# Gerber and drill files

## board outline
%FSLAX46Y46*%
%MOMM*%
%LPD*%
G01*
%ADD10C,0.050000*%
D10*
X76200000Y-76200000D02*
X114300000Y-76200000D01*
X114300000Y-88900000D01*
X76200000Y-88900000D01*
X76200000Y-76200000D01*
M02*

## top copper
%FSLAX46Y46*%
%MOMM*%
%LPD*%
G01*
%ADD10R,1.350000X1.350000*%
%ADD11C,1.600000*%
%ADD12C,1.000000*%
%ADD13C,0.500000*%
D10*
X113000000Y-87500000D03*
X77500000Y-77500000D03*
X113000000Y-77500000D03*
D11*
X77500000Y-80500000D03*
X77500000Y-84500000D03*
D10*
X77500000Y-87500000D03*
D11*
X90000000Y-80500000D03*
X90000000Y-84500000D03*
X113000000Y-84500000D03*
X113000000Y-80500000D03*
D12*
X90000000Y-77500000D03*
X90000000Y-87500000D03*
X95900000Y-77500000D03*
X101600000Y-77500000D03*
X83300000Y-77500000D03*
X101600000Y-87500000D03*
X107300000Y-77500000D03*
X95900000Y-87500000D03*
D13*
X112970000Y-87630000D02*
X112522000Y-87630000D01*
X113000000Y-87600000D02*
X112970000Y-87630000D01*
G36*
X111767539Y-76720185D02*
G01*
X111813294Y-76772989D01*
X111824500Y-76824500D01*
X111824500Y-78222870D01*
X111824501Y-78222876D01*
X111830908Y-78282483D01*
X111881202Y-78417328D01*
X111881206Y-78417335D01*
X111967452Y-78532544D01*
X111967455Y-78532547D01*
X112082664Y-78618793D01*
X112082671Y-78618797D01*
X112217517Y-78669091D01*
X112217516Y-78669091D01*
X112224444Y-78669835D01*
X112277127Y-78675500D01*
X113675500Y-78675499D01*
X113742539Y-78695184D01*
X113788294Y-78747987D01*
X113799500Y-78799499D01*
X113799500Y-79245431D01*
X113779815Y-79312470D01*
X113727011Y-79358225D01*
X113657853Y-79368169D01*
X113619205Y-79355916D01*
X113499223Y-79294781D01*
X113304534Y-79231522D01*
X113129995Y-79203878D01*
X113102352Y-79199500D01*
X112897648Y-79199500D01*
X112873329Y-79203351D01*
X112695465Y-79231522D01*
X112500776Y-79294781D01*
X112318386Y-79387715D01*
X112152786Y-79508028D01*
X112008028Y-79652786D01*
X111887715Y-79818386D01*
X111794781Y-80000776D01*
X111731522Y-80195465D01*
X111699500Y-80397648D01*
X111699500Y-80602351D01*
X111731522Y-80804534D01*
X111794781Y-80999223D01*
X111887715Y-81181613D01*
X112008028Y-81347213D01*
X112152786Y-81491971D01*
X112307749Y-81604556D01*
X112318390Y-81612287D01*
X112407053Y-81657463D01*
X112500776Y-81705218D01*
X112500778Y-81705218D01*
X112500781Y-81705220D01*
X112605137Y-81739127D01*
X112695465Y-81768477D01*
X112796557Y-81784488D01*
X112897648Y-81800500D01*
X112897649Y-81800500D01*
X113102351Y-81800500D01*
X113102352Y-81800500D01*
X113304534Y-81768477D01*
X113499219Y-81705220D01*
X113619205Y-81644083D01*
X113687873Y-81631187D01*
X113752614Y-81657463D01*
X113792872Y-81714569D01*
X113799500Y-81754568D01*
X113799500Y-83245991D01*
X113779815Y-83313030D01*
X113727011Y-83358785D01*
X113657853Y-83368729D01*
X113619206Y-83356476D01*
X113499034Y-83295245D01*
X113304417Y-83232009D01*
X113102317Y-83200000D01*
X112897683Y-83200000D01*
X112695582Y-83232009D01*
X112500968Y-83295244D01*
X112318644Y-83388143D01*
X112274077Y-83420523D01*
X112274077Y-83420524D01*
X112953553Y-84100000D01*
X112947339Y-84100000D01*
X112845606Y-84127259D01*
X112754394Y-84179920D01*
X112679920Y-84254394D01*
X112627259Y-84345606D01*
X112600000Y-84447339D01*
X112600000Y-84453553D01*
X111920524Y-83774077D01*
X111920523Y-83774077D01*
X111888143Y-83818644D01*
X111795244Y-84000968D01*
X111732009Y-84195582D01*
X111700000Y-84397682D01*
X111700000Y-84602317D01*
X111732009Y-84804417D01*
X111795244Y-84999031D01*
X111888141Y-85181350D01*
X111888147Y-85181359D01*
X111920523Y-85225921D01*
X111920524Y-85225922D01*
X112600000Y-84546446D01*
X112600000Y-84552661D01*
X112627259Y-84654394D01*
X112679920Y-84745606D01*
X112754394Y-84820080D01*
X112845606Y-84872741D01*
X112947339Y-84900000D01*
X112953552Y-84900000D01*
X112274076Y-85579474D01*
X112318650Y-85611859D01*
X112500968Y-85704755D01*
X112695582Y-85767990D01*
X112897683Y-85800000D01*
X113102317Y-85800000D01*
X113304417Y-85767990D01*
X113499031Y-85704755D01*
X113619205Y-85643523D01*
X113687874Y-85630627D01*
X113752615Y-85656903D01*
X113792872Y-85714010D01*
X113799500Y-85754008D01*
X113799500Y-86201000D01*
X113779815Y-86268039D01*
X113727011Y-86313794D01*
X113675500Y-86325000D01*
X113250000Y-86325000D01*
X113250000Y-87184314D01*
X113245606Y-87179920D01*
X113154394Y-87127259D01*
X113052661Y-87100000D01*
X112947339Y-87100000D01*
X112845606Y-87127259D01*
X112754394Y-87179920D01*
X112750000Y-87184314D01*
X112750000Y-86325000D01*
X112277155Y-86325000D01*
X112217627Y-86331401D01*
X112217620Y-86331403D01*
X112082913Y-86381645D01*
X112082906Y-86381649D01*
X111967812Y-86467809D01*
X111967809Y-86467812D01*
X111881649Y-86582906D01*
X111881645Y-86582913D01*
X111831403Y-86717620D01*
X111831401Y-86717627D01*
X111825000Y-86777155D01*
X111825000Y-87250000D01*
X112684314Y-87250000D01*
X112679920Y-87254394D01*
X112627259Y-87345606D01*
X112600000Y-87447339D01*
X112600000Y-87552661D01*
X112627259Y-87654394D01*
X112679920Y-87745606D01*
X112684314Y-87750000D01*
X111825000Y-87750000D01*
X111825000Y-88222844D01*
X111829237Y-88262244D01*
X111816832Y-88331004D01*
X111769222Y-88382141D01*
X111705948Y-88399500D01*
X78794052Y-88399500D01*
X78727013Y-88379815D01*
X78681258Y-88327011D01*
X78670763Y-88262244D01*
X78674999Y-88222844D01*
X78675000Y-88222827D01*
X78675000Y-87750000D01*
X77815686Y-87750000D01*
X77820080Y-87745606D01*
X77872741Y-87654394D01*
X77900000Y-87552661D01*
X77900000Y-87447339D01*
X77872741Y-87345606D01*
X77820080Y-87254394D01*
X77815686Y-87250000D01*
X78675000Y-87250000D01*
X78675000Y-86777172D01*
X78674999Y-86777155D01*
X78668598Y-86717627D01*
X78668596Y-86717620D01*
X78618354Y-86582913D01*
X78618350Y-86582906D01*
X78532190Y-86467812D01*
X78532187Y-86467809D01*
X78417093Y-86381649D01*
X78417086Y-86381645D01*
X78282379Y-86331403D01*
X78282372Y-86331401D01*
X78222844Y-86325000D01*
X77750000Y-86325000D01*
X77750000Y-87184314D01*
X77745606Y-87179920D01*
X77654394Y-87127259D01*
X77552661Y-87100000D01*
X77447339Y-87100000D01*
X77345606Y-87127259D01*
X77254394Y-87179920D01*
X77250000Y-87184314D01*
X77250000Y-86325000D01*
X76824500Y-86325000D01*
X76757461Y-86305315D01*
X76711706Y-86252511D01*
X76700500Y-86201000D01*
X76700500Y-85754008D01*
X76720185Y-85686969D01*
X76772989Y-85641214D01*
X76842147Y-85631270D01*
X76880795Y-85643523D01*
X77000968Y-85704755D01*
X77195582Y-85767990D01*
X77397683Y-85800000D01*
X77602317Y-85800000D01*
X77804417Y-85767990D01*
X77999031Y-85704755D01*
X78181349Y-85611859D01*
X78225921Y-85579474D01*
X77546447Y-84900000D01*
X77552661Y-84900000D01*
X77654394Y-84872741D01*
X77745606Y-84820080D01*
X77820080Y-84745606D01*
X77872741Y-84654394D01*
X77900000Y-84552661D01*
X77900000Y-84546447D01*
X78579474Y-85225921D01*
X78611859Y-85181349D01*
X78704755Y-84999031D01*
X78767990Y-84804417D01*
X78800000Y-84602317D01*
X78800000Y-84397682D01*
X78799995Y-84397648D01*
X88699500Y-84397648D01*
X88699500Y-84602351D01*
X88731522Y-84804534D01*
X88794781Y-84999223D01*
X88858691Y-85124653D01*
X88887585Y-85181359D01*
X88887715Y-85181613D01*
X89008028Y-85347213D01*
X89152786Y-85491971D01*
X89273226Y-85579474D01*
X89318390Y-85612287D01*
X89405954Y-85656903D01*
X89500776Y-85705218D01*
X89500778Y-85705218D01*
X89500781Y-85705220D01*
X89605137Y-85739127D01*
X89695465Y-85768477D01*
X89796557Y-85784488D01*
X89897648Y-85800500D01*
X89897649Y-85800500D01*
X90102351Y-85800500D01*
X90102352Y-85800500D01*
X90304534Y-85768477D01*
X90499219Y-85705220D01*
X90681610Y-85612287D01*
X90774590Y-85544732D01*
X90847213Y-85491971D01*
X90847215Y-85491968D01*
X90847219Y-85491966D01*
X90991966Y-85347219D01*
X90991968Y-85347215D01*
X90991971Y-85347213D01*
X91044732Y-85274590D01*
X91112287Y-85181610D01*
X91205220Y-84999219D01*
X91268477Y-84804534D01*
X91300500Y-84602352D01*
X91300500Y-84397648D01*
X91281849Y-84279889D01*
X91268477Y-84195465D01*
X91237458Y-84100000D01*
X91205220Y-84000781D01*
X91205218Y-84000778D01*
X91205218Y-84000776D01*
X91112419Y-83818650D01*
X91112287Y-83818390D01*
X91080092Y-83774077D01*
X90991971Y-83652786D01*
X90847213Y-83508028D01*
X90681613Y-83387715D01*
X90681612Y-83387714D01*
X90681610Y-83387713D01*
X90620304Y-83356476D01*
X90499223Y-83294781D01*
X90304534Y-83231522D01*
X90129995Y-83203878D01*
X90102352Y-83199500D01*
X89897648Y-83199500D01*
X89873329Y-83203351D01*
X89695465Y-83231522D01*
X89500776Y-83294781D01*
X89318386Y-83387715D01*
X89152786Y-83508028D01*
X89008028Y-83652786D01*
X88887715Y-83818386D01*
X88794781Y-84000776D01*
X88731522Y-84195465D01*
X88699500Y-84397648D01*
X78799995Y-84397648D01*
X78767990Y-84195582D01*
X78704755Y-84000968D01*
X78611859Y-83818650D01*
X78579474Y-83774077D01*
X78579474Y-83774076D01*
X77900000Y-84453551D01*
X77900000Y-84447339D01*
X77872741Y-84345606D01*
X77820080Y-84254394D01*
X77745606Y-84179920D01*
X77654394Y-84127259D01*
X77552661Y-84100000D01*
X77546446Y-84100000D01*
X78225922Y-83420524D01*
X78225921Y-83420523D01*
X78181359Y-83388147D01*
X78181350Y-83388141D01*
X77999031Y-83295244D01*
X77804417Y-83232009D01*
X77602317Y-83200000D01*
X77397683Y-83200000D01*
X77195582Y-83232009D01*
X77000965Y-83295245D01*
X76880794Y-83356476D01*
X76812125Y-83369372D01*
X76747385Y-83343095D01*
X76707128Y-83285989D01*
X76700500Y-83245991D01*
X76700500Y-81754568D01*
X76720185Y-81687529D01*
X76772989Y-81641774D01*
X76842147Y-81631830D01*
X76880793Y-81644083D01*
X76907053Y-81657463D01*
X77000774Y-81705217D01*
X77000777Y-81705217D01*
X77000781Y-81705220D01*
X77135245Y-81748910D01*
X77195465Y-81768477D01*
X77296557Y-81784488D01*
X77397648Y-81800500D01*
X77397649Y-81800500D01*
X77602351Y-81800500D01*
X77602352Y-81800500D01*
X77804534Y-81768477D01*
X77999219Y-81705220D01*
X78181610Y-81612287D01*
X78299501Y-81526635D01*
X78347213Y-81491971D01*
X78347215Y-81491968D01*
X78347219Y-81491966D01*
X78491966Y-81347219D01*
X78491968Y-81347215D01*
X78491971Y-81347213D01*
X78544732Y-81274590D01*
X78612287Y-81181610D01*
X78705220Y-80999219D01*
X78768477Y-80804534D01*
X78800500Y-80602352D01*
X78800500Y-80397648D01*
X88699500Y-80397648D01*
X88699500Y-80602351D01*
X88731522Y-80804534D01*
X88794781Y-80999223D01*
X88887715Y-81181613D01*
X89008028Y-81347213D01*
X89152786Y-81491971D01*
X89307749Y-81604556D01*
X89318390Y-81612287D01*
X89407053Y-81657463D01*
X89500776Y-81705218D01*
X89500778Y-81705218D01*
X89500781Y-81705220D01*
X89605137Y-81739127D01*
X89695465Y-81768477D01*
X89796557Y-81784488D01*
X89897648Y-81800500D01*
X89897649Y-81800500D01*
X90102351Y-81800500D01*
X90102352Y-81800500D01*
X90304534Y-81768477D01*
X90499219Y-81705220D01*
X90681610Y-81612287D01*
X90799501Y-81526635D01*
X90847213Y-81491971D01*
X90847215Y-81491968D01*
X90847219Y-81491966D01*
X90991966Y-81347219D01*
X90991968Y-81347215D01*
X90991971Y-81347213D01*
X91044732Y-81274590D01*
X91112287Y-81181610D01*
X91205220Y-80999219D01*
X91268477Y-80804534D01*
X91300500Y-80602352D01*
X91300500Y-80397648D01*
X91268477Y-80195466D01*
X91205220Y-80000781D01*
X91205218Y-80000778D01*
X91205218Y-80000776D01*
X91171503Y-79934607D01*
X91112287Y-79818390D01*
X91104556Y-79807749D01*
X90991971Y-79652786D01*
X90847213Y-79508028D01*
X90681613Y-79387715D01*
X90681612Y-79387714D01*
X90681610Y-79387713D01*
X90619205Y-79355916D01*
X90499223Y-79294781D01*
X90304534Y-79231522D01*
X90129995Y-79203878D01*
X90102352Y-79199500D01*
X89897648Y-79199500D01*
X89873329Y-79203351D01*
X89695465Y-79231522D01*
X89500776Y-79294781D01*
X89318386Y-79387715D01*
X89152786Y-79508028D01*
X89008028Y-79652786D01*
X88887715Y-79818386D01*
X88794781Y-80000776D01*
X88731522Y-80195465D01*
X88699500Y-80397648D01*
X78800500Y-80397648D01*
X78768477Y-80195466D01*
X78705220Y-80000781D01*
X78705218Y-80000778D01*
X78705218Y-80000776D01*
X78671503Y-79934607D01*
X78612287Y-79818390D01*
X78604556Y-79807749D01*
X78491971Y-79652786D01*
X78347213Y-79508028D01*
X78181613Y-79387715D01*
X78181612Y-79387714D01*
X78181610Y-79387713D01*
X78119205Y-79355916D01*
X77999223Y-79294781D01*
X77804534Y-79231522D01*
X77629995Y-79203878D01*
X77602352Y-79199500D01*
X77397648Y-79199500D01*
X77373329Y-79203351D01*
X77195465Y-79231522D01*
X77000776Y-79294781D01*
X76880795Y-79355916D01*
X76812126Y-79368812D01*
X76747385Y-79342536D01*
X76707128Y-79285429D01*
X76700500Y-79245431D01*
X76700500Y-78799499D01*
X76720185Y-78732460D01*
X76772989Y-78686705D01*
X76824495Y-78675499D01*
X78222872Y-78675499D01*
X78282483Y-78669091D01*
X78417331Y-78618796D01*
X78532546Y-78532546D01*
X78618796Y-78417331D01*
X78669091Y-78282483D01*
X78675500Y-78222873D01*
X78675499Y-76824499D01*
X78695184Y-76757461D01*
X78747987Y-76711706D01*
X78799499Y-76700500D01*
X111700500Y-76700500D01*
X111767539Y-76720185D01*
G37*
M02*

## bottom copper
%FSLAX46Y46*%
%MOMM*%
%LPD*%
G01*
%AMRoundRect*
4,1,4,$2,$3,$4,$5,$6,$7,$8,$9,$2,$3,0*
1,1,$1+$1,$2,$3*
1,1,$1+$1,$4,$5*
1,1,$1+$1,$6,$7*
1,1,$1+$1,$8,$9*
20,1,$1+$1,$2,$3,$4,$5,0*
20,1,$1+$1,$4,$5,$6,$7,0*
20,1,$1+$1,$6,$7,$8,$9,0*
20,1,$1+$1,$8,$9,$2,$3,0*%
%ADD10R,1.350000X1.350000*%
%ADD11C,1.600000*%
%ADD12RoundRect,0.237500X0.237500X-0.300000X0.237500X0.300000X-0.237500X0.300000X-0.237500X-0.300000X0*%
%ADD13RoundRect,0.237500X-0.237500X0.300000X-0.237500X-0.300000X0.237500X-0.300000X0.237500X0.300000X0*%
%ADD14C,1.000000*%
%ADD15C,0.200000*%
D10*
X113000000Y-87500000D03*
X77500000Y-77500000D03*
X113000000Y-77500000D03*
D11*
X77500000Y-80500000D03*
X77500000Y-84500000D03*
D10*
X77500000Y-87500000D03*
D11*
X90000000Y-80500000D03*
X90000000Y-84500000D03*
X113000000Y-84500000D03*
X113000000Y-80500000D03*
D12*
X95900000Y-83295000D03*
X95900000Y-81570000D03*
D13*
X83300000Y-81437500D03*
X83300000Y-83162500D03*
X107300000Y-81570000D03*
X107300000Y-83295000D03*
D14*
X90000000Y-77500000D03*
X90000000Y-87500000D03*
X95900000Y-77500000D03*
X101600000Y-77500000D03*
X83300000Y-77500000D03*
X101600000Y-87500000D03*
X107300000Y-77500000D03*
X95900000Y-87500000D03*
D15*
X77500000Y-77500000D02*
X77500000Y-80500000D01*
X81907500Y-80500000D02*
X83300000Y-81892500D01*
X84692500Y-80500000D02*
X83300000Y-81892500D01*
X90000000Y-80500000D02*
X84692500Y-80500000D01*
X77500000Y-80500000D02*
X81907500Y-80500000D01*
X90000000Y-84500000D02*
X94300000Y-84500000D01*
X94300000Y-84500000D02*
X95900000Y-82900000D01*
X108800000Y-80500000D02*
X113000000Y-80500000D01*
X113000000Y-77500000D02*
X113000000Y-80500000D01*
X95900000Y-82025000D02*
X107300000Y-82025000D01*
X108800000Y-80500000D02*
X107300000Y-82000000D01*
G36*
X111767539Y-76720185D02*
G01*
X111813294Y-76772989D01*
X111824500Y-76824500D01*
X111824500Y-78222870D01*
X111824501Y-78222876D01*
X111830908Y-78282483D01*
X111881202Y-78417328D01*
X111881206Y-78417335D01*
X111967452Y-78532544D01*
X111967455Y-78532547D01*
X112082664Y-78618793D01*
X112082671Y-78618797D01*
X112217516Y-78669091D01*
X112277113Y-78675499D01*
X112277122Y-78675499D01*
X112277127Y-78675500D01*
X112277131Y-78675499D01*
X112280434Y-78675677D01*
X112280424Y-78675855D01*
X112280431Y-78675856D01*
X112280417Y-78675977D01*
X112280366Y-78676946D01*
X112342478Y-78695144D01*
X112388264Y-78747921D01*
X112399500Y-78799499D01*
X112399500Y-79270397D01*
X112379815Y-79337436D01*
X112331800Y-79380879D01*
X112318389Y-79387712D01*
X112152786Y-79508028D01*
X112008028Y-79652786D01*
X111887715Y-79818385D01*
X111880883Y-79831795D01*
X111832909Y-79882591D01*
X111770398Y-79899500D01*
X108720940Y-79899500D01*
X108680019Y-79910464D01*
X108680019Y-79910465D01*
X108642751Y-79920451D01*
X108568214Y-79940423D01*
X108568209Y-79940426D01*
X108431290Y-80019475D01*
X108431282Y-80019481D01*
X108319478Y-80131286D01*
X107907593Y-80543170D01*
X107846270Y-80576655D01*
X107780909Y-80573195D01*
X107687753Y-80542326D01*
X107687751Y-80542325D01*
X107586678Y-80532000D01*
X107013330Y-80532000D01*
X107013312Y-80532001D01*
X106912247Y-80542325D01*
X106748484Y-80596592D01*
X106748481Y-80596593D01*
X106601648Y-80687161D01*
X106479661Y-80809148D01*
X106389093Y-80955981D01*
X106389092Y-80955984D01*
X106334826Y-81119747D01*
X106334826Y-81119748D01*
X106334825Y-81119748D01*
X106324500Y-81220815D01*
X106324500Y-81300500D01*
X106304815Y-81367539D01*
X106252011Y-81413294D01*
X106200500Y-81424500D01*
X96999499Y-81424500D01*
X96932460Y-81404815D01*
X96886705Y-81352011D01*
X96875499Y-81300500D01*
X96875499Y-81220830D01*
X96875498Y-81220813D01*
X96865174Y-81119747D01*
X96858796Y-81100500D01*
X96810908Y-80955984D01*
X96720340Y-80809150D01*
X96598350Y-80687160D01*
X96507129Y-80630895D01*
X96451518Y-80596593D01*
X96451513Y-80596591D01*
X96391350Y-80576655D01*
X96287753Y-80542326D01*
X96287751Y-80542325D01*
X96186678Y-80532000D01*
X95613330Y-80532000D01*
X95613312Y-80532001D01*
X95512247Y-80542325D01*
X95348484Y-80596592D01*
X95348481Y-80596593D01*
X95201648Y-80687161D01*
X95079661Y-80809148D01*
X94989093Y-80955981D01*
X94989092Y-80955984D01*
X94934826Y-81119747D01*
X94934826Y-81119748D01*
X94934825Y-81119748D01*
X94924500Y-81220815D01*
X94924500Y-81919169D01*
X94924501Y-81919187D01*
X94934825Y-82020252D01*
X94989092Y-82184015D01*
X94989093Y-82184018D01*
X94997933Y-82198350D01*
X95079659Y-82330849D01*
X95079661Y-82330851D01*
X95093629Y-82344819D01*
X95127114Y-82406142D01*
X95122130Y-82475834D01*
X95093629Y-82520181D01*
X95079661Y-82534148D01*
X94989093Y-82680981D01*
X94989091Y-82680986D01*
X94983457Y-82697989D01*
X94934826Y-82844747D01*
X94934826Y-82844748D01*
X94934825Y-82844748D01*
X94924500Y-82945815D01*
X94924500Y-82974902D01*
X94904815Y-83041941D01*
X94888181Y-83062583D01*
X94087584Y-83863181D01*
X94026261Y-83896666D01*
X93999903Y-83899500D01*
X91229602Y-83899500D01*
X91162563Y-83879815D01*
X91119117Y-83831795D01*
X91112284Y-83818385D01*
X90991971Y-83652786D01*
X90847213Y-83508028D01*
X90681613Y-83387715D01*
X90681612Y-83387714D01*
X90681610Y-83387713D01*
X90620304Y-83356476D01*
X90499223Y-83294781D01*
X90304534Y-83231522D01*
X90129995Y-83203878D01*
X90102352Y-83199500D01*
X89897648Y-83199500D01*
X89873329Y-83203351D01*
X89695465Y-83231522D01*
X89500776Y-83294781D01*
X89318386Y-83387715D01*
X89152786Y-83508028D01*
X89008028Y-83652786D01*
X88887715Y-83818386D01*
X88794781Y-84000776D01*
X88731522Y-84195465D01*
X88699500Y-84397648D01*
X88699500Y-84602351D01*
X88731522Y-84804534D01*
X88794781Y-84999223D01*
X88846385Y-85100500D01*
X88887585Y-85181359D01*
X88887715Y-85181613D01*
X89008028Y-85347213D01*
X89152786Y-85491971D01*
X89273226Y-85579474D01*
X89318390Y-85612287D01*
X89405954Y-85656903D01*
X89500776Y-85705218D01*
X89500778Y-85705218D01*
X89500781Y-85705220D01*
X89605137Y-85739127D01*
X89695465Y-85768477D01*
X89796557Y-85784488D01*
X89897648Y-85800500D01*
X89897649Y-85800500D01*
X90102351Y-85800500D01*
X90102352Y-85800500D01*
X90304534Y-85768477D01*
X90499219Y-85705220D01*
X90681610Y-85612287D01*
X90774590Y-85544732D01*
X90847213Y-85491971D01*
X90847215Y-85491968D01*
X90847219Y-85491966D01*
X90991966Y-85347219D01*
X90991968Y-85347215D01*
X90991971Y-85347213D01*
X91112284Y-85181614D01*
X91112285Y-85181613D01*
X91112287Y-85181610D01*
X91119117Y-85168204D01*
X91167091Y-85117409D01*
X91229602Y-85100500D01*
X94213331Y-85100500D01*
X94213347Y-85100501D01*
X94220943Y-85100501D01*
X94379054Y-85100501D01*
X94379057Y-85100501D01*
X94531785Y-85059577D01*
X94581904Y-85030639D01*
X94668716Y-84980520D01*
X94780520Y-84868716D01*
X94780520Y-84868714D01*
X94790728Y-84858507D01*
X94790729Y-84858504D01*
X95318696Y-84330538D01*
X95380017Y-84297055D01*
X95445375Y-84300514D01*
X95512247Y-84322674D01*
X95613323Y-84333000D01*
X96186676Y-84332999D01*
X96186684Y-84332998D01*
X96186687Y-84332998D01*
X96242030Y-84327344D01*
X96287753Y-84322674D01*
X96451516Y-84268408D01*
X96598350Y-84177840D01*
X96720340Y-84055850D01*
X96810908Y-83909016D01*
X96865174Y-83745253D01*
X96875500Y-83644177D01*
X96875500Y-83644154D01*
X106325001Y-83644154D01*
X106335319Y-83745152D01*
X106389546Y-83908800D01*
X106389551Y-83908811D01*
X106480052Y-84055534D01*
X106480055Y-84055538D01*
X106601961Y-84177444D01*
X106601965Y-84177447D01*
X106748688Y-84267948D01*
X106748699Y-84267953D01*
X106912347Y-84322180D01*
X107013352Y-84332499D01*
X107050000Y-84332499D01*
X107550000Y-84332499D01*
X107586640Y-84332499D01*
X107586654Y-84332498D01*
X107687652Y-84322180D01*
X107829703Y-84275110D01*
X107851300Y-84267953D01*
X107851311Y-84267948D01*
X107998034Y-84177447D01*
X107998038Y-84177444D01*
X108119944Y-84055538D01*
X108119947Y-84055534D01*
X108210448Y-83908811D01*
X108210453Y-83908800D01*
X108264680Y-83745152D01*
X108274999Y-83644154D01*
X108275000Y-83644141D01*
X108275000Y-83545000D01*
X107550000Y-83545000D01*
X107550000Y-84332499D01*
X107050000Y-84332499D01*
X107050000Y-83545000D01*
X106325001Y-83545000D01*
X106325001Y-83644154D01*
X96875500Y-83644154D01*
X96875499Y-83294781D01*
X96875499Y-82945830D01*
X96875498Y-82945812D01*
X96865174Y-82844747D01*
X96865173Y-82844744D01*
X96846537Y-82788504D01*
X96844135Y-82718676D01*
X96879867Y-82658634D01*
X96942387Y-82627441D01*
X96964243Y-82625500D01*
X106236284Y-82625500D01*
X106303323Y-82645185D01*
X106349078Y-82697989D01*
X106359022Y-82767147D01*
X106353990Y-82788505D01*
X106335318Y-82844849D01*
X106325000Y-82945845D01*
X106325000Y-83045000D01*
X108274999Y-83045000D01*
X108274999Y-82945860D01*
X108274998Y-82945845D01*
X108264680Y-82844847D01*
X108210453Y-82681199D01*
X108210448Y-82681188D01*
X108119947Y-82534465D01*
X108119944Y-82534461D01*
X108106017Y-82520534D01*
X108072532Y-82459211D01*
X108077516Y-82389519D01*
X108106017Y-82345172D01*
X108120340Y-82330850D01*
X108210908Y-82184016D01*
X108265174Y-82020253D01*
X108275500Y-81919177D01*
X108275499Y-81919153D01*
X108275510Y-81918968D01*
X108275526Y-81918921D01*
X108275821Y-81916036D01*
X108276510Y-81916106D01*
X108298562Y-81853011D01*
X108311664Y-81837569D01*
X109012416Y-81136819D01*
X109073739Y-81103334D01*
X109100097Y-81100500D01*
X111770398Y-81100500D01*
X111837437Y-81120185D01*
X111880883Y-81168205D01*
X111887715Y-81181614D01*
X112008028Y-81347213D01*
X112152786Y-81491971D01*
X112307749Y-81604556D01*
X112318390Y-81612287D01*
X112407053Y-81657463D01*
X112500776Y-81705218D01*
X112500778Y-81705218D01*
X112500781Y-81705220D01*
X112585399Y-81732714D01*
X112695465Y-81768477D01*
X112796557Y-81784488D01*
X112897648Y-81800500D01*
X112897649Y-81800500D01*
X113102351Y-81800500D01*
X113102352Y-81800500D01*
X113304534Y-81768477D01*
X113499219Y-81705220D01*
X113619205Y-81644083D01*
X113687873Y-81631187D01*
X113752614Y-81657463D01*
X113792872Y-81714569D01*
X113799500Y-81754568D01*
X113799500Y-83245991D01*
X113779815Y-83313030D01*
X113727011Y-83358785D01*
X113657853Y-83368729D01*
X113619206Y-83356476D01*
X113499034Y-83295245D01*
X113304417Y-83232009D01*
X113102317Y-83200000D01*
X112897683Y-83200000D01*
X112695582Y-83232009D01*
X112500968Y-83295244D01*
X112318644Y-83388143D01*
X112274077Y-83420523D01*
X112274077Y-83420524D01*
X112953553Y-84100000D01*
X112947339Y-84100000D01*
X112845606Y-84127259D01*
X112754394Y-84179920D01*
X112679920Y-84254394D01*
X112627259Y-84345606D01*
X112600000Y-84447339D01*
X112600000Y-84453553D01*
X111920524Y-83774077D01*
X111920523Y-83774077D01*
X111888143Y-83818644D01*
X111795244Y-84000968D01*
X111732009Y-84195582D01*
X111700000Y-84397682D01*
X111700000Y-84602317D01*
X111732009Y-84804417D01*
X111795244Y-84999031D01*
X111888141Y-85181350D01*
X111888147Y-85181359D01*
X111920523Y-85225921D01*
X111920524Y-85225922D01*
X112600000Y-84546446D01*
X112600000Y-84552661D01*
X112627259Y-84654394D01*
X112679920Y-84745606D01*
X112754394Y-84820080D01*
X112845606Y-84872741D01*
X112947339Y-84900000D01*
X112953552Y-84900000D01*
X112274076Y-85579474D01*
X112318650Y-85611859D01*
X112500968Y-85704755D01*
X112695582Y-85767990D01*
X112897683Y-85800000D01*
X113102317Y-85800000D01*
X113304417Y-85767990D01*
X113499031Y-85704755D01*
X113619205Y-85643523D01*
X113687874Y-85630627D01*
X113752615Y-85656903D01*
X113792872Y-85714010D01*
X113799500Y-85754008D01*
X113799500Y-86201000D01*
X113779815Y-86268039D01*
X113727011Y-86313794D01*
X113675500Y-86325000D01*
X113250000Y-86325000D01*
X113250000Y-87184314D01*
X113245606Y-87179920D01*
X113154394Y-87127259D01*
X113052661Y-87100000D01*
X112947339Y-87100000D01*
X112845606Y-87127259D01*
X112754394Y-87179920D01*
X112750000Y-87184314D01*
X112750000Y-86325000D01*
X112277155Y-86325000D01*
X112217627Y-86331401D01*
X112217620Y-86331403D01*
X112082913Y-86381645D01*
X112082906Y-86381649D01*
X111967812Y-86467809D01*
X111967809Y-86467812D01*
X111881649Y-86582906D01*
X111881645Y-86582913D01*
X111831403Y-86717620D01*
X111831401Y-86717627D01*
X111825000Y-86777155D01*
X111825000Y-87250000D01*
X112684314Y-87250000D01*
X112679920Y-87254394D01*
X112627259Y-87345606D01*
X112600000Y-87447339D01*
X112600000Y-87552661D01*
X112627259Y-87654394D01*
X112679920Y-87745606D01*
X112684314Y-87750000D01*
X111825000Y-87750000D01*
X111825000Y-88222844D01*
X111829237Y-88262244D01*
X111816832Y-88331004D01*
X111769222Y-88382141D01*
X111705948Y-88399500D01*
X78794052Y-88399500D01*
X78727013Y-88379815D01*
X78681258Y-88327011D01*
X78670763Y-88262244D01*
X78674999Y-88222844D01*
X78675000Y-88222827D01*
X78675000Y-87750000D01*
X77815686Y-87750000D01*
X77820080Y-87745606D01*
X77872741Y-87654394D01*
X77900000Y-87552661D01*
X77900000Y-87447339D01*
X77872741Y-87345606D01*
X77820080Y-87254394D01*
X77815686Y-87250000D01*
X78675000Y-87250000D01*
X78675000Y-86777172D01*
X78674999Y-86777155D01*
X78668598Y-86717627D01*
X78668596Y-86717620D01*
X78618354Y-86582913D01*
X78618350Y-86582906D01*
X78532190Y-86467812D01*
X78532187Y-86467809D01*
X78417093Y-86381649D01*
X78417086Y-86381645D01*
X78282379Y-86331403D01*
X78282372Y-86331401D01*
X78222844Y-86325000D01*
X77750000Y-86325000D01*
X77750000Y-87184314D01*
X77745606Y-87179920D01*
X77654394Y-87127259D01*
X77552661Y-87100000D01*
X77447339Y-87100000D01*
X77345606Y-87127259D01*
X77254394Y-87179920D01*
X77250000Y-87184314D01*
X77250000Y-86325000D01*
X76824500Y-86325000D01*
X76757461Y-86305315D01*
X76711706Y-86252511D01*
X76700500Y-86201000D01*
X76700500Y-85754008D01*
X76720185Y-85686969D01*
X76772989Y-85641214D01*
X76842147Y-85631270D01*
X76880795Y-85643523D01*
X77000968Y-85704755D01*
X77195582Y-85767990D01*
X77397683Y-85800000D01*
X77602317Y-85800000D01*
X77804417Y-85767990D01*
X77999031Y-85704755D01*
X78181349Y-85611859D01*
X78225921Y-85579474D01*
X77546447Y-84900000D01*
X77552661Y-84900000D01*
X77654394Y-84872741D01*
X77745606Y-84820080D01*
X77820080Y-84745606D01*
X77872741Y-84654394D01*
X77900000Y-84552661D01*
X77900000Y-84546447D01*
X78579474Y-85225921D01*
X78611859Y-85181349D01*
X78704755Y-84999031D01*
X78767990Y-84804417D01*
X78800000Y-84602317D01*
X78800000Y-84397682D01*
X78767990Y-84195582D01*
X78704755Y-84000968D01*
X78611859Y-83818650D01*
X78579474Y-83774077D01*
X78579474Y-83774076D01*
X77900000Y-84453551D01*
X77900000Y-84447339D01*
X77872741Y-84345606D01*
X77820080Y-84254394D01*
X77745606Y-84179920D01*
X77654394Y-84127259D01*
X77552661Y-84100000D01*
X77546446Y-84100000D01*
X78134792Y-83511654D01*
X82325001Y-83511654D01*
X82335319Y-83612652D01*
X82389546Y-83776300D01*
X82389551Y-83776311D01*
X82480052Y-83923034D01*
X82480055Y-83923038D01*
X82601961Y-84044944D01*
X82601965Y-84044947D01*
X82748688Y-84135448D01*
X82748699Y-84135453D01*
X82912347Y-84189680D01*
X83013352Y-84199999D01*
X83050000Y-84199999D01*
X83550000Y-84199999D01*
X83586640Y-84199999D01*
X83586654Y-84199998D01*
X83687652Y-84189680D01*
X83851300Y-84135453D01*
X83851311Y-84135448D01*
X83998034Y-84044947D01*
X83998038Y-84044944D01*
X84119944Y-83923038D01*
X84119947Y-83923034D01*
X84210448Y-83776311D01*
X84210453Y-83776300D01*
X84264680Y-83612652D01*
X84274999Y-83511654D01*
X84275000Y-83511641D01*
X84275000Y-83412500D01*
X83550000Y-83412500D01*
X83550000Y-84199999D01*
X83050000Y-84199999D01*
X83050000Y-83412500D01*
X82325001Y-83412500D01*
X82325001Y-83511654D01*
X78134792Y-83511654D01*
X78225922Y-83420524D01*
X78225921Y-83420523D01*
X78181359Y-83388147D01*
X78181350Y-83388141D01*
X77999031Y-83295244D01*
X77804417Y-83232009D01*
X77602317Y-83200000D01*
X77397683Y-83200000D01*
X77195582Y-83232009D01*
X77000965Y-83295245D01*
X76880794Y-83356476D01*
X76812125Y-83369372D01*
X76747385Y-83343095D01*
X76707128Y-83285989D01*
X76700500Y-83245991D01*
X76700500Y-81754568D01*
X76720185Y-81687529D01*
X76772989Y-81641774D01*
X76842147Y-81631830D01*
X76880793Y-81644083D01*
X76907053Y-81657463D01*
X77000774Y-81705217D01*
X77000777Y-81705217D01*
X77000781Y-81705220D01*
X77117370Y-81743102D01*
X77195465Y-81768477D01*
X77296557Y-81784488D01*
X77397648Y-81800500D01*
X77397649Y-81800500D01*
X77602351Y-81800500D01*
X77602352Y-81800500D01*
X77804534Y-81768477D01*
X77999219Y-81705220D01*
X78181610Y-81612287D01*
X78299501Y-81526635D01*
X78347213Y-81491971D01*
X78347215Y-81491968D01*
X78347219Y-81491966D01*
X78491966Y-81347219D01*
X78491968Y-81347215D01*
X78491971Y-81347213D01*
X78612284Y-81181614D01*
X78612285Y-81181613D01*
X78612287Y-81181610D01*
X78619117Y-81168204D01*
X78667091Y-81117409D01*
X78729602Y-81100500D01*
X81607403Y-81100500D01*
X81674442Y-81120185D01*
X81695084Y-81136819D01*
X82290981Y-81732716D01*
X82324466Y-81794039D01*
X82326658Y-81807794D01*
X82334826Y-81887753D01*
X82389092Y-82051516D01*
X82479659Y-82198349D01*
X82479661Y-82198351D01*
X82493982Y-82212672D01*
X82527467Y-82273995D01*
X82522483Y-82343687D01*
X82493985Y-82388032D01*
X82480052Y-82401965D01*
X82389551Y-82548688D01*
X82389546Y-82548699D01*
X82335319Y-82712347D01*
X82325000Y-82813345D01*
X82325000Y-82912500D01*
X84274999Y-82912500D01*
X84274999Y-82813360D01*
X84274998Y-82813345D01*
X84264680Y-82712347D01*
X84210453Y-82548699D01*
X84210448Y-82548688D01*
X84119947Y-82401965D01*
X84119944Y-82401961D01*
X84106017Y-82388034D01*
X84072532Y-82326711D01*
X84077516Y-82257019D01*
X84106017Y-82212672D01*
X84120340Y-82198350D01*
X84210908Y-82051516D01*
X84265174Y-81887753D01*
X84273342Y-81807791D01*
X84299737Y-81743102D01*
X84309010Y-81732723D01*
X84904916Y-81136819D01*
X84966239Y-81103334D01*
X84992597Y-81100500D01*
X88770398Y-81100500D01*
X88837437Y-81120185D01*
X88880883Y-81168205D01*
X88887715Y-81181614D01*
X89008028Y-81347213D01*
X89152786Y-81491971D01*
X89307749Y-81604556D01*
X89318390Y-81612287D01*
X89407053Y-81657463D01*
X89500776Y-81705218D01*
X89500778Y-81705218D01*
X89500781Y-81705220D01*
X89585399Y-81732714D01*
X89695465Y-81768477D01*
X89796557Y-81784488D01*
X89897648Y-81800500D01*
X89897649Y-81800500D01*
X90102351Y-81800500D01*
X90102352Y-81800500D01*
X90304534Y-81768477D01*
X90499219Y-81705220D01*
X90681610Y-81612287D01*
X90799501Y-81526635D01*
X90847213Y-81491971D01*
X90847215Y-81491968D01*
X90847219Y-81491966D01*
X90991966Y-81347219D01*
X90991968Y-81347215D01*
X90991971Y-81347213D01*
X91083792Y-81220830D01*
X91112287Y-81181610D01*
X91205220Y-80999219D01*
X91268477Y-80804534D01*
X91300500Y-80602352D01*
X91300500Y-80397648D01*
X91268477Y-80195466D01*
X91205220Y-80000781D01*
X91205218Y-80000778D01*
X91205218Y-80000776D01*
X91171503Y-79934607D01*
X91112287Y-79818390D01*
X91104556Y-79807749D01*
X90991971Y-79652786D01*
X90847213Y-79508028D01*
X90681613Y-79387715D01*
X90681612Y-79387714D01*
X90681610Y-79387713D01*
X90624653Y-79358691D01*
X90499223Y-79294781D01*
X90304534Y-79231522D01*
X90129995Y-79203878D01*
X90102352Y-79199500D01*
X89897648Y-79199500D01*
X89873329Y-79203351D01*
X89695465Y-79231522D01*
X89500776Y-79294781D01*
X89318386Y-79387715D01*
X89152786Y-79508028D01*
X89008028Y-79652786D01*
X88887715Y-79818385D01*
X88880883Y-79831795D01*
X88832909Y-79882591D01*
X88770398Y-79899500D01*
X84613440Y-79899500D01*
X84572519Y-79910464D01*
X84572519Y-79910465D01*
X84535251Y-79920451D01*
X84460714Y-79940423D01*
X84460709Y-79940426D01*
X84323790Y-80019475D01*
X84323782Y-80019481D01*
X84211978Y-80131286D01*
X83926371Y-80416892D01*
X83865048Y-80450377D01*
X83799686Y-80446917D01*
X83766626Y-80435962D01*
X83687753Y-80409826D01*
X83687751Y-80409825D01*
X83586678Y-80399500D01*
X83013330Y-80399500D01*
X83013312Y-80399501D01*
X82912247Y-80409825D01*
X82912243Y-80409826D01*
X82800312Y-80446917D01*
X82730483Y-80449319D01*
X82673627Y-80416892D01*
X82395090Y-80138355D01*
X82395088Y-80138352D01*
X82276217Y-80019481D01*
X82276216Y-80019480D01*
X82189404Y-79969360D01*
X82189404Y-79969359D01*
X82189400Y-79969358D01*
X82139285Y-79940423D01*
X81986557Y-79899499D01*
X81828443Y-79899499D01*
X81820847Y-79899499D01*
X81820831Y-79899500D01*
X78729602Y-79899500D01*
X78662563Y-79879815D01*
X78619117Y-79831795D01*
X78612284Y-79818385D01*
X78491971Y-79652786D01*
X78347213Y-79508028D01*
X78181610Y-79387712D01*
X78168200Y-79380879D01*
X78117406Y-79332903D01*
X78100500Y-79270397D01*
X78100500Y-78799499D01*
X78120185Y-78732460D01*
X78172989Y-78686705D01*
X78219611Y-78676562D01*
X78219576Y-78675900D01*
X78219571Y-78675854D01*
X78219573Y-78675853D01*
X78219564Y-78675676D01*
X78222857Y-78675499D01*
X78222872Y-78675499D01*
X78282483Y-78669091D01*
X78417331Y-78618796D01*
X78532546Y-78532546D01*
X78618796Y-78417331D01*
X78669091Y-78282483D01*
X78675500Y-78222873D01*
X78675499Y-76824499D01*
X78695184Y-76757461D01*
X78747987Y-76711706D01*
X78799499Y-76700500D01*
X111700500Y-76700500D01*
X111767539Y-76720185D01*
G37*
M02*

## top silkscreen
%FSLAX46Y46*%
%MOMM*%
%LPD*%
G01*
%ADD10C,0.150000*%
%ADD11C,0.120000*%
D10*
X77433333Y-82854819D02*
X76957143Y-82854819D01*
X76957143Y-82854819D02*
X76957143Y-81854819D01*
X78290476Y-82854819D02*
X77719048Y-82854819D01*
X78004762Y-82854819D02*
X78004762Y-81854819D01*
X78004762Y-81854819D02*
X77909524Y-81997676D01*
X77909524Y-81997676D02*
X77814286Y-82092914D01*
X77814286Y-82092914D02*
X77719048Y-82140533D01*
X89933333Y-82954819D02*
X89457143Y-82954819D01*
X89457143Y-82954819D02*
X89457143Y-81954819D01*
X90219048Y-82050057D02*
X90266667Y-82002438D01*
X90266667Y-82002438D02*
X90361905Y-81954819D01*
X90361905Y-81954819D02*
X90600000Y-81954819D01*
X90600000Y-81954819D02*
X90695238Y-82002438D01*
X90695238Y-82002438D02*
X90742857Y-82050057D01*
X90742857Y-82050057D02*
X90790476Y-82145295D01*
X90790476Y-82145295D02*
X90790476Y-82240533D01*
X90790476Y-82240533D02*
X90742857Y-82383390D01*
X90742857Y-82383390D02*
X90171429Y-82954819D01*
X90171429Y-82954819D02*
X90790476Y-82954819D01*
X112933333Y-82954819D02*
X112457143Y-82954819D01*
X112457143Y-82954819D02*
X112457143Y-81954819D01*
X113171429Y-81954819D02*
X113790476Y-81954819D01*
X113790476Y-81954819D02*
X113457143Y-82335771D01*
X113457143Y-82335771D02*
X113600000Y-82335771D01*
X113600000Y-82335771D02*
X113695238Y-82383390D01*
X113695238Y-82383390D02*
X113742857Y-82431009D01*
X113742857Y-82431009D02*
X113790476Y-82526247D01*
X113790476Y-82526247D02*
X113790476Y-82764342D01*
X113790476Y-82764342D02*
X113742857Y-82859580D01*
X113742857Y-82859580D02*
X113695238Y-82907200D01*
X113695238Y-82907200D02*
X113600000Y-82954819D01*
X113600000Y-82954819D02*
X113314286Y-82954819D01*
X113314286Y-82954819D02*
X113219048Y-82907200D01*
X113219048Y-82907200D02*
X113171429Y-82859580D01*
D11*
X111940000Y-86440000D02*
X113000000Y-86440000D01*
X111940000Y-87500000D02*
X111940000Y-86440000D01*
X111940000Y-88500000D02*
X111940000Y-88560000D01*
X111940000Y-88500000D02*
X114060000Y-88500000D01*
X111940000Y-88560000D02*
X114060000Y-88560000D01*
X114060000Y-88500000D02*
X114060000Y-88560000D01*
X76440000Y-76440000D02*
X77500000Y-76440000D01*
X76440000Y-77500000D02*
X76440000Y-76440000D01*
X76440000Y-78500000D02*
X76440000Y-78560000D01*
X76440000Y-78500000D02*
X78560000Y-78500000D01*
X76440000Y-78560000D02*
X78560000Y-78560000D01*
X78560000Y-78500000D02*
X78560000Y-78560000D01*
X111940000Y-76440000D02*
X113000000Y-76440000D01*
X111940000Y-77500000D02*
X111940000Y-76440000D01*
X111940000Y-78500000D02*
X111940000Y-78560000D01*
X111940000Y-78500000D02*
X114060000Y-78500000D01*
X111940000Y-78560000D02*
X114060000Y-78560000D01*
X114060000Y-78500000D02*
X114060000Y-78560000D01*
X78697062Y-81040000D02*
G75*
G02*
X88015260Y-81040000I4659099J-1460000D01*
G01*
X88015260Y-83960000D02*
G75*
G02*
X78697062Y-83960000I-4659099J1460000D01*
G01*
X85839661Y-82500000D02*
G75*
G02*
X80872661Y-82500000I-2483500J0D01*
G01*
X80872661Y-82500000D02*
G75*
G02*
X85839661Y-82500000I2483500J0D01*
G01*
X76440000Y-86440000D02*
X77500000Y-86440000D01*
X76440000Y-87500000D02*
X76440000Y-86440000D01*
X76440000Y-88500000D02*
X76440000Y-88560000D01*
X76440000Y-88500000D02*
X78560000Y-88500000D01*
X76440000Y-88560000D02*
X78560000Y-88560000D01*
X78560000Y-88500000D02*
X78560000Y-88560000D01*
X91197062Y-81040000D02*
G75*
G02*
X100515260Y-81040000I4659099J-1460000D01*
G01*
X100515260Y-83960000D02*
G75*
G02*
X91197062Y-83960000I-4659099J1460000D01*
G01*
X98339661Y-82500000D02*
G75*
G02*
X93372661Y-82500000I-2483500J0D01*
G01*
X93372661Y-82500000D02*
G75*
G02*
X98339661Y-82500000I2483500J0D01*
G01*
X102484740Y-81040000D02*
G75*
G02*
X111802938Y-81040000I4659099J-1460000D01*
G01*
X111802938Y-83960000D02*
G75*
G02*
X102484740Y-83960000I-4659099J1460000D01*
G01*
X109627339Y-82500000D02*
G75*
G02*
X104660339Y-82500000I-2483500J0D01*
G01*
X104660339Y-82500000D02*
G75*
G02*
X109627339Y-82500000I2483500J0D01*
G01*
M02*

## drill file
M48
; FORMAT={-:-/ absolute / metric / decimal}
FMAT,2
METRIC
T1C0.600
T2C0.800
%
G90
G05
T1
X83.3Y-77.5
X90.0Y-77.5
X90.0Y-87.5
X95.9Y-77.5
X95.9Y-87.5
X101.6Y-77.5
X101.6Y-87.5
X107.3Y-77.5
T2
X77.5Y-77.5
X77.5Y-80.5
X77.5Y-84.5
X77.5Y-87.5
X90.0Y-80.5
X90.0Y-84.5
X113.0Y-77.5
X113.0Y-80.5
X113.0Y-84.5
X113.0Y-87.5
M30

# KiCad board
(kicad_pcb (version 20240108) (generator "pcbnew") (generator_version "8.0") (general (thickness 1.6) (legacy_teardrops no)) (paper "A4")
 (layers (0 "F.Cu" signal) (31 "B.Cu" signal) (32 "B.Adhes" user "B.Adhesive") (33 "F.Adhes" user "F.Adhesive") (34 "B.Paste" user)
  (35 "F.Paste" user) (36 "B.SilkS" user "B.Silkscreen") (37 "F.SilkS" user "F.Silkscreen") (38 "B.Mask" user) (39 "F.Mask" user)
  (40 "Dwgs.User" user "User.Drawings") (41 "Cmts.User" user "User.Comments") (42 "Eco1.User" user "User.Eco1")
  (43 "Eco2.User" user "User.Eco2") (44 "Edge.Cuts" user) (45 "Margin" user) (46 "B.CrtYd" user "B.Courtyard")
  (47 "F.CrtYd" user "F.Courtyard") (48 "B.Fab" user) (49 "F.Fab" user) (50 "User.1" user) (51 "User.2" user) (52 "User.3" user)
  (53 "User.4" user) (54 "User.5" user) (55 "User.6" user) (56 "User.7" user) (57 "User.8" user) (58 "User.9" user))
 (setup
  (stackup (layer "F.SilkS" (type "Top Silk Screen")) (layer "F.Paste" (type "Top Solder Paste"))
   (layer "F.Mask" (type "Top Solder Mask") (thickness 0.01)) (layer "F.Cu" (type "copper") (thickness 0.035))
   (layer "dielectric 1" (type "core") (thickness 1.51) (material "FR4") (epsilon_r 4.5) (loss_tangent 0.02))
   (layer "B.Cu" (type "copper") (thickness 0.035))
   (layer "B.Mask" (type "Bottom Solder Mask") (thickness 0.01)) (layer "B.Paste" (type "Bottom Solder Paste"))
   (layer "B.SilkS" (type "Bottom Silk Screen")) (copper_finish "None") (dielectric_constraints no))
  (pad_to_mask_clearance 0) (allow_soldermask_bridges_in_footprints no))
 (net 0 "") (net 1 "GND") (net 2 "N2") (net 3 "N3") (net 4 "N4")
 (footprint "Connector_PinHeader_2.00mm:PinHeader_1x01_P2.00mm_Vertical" (layer "F.Cu") (at 113 87.5)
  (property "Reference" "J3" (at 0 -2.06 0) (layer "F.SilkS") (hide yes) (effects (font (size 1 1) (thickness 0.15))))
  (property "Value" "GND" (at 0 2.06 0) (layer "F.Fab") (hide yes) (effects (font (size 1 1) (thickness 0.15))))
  (fp_line (start -1.06 -1.06) (end 0 -1.06) (stroke (width 0.12) (type solid)) (layer "F.SilkS"))
  (fp_line (start -1.06 0) (end -1.06 -1.06) (stroke (width 0.12) (type solid)) (layer "F.SilkS"))
  (fp_line (start -1.06 1) (end -1.06 1.06) (stroke (width 0.12) (type solid)) (layer "F.SilkS"))
  (fp_line (start -1.06 1) (end 1.06 1) (stroke (width 0.12) (type solid)) (layer "F.SilkS"))
  (fp_line (start -1.06 1.06) (end 1.06 1.06) (stroke (width 0.12) (type solid)) (layer "F.SilkS"))
  (fp_line (start 1.06 1) (end 1.06 1.06) (stroke (width 0.12) (type solid)) (layer "F.SilkS"))
  (pad "1" thru_hole rect (at 0 0) (size 1.35 1.35) (drill 0.8) (layers "*.Cu" "*.Mask") (remove_unused_layers no) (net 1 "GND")))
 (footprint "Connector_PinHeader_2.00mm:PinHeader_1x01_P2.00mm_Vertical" (layer "F.Cu") (at 77.5 77.5)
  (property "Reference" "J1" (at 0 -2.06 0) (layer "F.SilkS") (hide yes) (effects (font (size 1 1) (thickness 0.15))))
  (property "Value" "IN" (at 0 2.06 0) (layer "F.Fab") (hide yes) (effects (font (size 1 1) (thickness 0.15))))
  (fp_line (start -1.06 -1.06) (end 0 -1.06) (stroke (width 0.12) (type solid)) (layer "F.SilkS"))
  (fp_line (start -1.06 0) (end -1.06 -1.06) (stroke (width 0.12) (type solid)) (layer "F.SilkS"))
  (fp_line (start -1.06 1) (end -1.06 1.06) (stroke (width 0.12) (type solid)) (layer "F.SilkS"))
  (fp_line (start -1.06 1) (end 1.06 1) (stroke (width 0.12) (type solid)) (layer "F.SilkS"))
  (fp_line (start -1.06 1.06) (end 1.06 1.06) (stroke (width 0.12) (type solid)) (layer "F.SilkS"))
  (fp_line (start 1.06 1) (end 1.06 1.06) (stroke (width 0.12) (type solid)) (layer "F.SilkS"))
  (pad "1" thru_hole rect (at 0 0) (size 1.35 1.35) (drill 0.8) (layers "*.Cu" "*.Mask") (remove_unused_layers no) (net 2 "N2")))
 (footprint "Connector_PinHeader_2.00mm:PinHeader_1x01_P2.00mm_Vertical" (layer "F.Cu") (at 113 77.5)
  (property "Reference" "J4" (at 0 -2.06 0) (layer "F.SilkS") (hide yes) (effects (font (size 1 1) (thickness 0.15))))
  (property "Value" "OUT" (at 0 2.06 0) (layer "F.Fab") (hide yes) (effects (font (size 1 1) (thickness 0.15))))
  (fp_line (start -1.06 -1.06) (end 0 -1.06) (stroke (width 0.12) (type solid)) (layer "F.SilkS"))
  (fp_line (start -1.06 0) (end -1.06 -1.06) (stroke (width 0.12) (type solid)) (layer "F.SilkS"))
  (fp_line (start -1.06 1) (end -1.06 1.06) (stroke (width 0.12) (type solid)) (layer "F.SilkS"))
  (fp_line (start -1.06 1) (end 1.06 1) (stroke (width 0.12) (type solid)) (layer "F.SilkS"))
  (fp_line (start -1.06 1.06) (end 1.06 1.06) (stroke (width 0.12) (type solid)) (layer "F.SilkS"))
  (fp_line (start 1.06 1) (end 1.06 1.06) (stroke (width 0.12) (type solid)) (layer "F.SilkS"))
  (pad "1" thru_hole rect (at 0 0) (size 1.35 1.35) (drill 0.8) (layers "*.Cu" "*.Mask") (remove_unused_layers no) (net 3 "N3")))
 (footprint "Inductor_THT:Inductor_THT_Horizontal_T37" (layer "F.Cu") (at 77.5 82.5)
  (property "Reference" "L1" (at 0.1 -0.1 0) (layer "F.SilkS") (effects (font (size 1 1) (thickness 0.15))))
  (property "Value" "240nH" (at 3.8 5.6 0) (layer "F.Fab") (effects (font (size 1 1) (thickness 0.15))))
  (fp_arc (start 1.197062 -1.46) (mid 5.856161 -4.8825) (end 10.51526 -1.46) (stroke (width 0.12) (type solid)) (layer "F.SilkS"))
  (fp_arc (start 10.51526 1.46) (mid 5.856161 4.8825) (end 1.197062 1.46) (stroke (width 0.12) (type solid)) (layer "F.SilkS"))
  (fp_circle (center 5.856161 0) (end 8.339661 0) (stroke (width 0.12) (type solid)) (fill none) (layer "F.SilkS"))
  (pad "1" thru_hole circle (at 0 -2) (size 1.6 1.6) (drill 0.8) (layers "*.Cu" "*.Mask") (remove_unused_layers no) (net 2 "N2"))
  (pad "2" thru_hole circle (at 0 2) (size 1.6 1.6) (drill 0.8) (layers "*.Cu" "*.Mask") (remove_unused_layers no) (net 1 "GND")))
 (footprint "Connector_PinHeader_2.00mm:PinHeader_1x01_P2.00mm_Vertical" (layer "F.Cu") (at 77.5 87.5)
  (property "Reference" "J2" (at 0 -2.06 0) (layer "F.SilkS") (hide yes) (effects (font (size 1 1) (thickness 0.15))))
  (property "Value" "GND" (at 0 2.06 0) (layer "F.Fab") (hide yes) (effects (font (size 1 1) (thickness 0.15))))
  (fp_line (start -1.06 -1.06) (end 0 -1.06) (stroke (width 0.12) (type solid)) (layer "F.SilkS"))
  (fp_line (start -1.06 0) (end -1.06 -1.06) (stroke (width 0.12) (type solid)) (layer "F.SilkS"))
  (fp_line (start -1.06 1) (end -1.06 1.06) (stroke (width 0.12) (type solid)) (layer "F.SilkS"))
  (fp_line (start -1.06 1) (end 1.06 1) (stroke (width 0.12) (type solid)) (layer "F.SilkS"))
  (fp_line (start -1.06 1.06) (end 1.06 1.06) (stroke (width 0.12) (type solid)) (layer "F.SilkS"))
  (fp_line (start 1.06 1) (end 1.06 1.06) (stroke (width 0.12) (type solid)) (layer "F.SilkS"))
  (pad "1" thru_hole rect (at 0 0) (size 1.35 1.35) (drill 0.8) (layers "*.Cu" "*.Mask") (remove_unused_layers no) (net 1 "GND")))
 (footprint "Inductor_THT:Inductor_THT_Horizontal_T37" (layer "F.Cu") (at 90 82.5)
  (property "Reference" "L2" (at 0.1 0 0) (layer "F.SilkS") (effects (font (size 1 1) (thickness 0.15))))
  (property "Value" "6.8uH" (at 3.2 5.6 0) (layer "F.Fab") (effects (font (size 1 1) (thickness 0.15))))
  (fp_arc (start 1.197062 -1.46) (mid 5.856161 -4.8825) (end 10.51526 -1.46) (stroke (width 0.12) (type solid)) (layer "F.SilkS"))
  (fp_arc (start 10.51526 1.46) (mid 5.856161 4.8825) (end 1.197062 1.46) (stroke (width 0.12) (type solid)) (layer "F.SilkS"))
  (fp_circle (center 5.856161 0) (end 8.339661 0) (stroke (width 0.12) (type solid)) (fill none) (layer "F.SilkS"))
  (pad "1" thru_hole circle (at 0 -2) (size 1.6 1.6) (drill 0.8) (layers "*.Cu" "*.Mask") (remove_unused_layers no) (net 2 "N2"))
  (pad "2" thru_hole circle (at 0 2) (size 1.6 1.6) (drill 0.8) (layers "*.Cu" "*.Mask") (remove_unused_layers no) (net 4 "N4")))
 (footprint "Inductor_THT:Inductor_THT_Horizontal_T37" (layer "F.Cu") (at 113 82.5 180)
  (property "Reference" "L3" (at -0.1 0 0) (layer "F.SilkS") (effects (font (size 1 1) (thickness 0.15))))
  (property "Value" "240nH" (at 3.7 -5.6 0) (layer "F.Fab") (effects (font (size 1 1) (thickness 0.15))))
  (fp_arc (start 10.51526 1.46) (mid 5.856161 4.8825) (end 1.197062 1.46) (stroke (width 0.12) (type solid)) (layer "F.SilkS"))
  (fp_arc (start 1.197062 -1.46) (mid 5.856161 -4.8825) (end 10.51526 -1.46) (stroke (width 0.12) (type solid)) (layer "F.SilkS"))
  (fp_circle (center 5.856161 0) (end 8.339661 0) (stroke (width 0.12) (type solid)) (fill none) (layer "F.SilkS"))
  (pad "1" thru_hole circle (at 0 -2 180) (size 1.6 1.6) (drill 0.8) (layers "*.Cu" "*.Mask") (remove_unused_layers no) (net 1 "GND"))
  (pad "2" thru_hole circle (at 0 2 180) (size 1.6 1.6) (drill 0.8) (layers "*.Cu" "*.Mask") (remove_unused_layers no) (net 3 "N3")))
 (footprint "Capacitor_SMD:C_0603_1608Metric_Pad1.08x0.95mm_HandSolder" (layer "B.Cu") (at 95.9 82.4325 90)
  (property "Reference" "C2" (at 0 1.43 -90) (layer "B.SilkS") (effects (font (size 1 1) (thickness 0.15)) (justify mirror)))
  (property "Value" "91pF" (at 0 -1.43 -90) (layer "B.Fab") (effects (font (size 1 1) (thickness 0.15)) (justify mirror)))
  (pad "1" smd roundrect (at -0.8625 0 90) (size 1.075 0.95) (layers "B.Cu" "B.Paste" "B.Mask") (roundrect_rratio 0.25) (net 4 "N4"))
  (pad "2" smd roundrect (at 0.8625 0 90) (size 1.075 0.95) (layers "B.Cu" "B.Paste" "B.Mask") (roundrect_rratio 0.25) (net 3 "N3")))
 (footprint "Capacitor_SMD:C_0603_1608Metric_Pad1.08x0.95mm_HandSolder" (layer "B.Cu") (at 83.3 82.3 -90)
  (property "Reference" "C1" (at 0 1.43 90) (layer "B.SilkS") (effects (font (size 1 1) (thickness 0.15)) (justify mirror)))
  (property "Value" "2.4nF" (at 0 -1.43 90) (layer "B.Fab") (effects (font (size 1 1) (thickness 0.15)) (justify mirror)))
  (pad "1" smd roundrect (at -0.8625 0 270) (size 1.075 0.95) (layers "B.Cu" "B.Paste" "B.Mask") (roundrect_rratio 0.25) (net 2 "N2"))
  (pad "2" smd roundrect (at 0.8625 0 270) (size 1.075 0.95) (layers "B.Cu" "B.Paste" "B.Mask") (roundrect_rratio 0.25) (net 1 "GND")))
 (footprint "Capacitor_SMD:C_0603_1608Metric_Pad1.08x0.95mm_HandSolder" (layer "B.Cu") (at 107.3 82.4325 -90)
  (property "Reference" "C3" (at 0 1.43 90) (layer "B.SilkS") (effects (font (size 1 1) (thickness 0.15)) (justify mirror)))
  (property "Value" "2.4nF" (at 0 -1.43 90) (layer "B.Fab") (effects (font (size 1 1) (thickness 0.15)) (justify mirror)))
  (pad "1" smd roundrect (at -0.8625 0 270) (size 1.075 0.95) (layers "B.Cu" "B.Paste" "B.Mask") (roundrect_rratio 0.25) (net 3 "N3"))
  (pad "2" smd roundrect (at 0.8625 0 270) (size 1.075 0.95) (layers "B.Cu" "B.Paste" "B.Mask") (roundrect_rratio 0.25) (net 1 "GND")))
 (gr_rect (start 76.2 76.2) (end 114.3 88.9) (stroke (width 0.05) (type default)) (fill none) (layer "Edge.Cuts"))
 (segment (start 112.97 87.63) (end 112.522 87.63) (width 0.5) (layer "F.Cu") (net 1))
 (segment (start 113 87.6) (end 112.97 87.63) (width 0.5) (layer "F.Cu") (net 1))
 (via (at 90 77.5) (size 1) (drill 0.6) (layers "F.Cu" "B.Cu") (free yes) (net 1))
 (via (at 90 87.5) (size 1) (drill 0.6) (layers "F.Cu" "B.Cu") (free yes) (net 1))
 (via (at 95.9 77.5) (size 1) (drill 0.6) (layers "F.Cu" "B.Cu") (free yes) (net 1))
 (via (at 101.6 77.5) (size 1) (drill 0.6) (layers "F.Cu" "B.Cu") (free yes) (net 1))
 (via (at 83.3 77.5) (size 1) (drill 0.6) (layers "F.Cu" "B.Cu") (free yes) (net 1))
 (via (at 101.6 87.5) (size 1) (drill 0.6) (layers "F.Cu" "B.Cu") (free yes) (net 1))
 (via (at 107.3 77.5) (size 1) (drill 0.6) (layers "F.Cu" "B.Cu") (free yes) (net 1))
 (via (at 95.9 87.5) (size 1) (drill 0.6) (layers "F.Cu" "B.Cu") (free yes) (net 1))
 (segment (start 77.5 77.5) (end 77.5 80.5) (width 0.2) (layer "B.Cu") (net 2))
 (segment (start 81.9075 80.5) (end 83.3 81.8925) (width 0.2) (layer "B.Cu") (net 2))
 (segment (start 84.6925 80.5) (end 83.3 81.8925) (width 0.2) (layer "B.Cu") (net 2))
 (segment (start 90 80.5) (end 84.6925 80.5) (width 0.2) (layer "B.Cu") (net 2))
 (segment (start 77.5 80.5) (end 81.9075 80.5) (width 0.2) (layer "B.Cu") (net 2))
 (segment (start 90 84.5) (end 94.3 84.5) (width 0.2) (layer "B.Cu") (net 4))
 (segment (start 94.3 84.5) (end 95.9 82.9) (width 0.2) (layer "B.Cu") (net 4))
 (segment (start 108.8 80.5) (end 113 80.5) (width 0.2) (layer "B.Cu") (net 3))
 (segment (start 113 77.5) (end 113 80.5) (width 0.2) (layer "B.Cu") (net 3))
 (segment (start 95.9 82.025) (end 107.3 82.025) (width 0.2) (layer "B.Cu") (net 3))
 (segment (start 108.8 80.5) (end 107.3 82) (width 0.2) (layer "B.Cu") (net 3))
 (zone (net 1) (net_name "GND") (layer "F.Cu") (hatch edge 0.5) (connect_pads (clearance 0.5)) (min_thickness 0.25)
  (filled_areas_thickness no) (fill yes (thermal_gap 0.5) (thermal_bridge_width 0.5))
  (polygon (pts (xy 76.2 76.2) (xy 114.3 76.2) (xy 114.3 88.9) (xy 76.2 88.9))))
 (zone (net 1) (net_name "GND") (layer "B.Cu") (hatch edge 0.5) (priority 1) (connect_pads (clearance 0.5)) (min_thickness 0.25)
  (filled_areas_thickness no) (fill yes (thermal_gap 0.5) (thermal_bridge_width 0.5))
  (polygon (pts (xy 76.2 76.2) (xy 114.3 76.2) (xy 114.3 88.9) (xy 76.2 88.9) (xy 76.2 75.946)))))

